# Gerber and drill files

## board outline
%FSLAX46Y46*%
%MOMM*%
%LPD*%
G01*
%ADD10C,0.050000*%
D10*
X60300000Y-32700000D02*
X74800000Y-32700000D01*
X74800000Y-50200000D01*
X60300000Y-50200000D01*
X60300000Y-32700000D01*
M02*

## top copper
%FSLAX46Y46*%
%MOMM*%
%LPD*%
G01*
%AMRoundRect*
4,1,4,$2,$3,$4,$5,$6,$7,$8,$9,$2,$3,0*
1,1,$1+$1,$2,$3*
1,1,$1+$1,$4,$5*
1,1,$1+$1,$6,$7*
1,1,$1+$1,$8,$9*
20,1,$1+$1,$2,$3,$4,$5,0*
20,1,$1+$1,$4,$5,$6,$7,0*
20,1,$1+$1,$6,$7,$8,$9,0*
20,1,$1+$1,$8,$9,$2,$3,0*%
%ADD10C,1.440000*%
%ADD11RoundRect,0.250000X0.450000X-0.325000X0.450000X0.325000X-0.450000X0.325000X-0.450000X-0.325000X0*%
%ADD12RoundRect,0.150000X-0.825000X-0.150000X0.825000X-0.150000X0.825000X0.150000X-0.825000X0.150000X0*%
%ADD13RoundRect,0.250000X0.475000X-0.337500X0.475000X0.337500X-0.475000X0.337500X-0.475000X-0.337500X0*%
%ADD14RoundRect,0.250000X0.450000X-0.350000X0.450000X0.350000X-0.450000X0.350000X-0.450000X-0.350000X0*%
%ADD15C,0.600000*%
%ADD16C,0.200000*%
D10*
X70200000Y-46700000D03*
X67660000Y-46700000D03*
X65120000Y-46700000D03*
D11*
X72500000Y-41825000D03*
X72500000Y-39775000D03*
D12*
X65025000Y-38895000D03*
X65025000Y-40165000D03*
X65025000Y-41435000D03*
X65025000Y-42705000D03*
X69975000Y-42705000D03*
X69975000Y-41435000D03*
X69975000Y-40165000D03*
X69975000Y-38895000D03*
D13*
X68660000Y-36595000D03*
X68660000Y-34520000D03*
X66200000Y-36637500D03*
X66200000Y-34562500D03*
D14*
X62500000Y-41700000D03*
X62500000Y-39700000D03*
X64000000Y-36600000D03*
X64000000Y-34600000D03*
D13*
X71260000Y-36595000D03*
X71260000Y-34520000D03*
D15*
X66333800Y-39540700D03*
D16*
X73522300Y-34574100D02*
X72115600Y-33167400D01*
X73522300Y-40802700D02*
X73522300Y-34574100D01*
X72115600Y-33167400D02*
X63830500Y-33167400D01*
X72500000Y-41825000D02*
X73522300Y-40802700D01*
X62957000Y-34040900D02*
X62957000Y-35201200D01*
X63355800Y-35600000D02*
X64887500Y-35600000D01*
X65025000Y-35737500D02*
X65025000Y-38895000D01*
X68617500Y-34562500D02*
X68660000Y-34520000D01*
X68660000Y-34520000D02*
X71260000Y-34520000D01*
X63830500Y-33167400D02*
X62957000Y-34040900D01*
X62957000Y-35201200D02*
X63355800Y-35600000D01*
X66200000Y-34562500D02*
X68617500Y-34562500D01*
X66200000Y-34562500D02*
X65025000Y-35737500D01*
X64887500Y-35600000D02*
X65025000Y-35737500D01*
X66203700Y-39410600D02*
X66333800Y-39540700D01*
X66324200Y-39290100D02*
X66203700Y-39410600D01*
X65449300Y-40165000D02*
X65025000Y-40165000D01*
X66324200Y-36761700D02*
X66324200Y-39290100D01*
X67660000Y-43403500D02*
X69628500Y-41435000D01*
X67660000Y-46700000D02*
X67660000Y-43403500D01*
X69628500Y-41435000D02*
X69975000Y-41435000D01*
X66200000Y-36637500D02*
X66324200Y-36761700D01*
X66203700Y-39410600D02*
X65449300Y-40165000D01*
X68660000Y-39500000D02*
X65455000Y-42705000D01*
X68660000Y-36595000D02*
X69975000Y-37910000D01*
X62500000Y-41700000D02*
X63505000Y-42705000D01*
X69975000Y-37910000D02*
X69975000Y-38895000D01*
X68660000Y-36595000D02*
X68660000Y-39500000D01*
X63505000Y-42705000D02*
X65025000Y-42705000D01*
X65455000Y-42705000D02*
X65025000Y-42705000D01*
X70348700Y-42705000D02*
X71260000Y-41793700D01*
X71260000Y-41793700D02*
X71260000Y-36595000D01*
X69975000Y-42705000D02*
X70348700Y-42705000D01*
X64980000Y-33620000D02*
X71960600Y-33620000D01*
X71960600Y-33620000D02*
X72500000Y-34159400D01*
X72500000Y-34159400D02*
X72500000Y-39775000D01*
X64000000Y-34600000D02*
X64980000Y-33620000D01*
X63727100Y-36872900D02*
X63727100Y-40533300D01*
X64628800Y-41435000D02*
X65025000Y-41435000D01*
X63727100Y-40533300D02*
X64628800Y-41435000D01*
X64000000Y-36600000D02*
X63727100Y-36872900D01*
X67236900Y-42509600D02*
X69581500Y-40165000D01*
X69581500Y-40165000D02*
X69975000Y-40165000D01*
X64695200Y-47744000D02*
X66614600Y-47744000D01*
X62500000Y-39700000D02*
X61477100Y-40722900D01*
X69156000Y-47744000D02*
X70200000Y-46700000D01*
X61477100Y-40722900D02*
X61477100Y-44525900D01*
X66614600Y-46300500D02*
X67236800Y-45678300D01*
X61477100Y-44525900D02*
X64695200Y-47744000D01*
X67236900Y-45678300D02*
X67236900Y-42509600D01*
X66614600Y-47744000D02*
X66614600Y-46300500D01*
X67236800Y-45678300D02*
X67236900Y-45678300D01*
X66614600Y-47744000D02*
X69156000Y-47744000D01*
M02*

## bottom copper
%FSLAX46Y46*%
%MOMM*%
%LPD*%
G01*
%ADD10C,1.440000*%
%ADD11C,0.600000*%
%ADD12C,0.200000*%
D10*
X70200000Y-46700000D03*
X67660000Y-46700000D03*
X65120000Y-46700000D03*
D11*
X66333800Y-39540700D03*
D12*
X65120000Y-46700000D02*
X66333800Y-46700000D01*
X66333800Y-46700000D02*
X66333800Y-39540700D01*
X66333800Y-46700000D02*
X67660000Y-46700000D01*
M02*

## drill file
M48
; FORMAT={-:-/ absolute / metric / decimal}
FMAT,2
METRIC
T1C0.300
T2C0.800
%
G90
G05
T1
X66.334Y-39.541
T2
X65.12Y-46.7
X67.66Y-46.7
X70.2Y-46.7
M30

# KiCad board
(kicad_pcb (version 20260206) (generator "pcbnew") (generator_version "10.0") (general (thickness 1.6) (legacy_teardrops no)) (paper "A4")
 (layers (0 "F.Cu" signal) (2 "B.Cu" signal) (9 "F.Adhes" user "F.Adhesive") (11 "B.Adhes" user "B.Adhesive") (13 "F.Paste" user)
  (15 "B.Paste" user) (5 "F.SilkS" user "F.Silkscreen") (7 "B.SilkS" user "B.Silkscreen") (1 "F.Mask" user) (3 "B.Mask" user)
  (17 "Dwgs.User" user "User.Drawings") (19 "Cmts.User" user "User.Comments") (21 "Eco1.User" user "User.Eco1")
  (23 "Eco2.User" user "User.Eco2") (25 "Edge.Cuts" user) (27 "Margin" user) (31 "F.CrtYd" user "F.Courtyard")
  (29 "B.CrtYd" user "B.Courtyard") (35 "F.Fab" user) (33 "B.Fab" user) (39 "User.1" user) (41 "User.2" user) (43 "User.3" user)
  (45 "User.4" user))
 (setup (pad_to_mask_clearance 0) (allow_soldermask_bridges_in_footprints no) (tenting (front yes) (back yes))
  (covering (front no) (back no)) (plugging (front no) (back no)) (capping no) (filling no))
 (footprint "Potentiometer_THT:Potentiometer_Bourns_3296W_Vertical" (layer "F.Cu") (at 70.2 46.7)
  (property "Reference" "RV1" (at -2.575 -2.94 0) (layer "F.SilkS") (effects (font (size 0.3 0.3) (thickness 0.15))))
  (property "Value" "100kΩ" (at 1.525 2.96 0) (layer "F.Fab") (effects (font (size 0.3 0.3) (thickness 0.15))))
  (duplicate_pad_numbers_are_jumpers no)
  (pad "1" thru_hole circle (at 0 0) (size 1.44 1.44) (drill 0.8) (layers "*.Cu" "*.Mask") (remove_unused_layers no) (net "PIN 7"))
  (pad "2" thru_hole circle (at -2.54 0) (size 1.44 1.44) (drill 0.8) (layers "*.Cu" "*.Mask") (remove_unused_layers no) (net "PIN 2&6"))
  (pad "3" thru_hole circle (at -5.08 0) (size 1.44 1.44) (drill 0.8) (layers "*.Cu" "*.Mask") (remove_unused_layers no) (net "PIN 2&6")))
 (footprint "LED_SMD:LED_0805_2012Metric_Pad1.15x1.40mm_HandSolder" (layer "F.Cu") (at 72.5 40.8 90)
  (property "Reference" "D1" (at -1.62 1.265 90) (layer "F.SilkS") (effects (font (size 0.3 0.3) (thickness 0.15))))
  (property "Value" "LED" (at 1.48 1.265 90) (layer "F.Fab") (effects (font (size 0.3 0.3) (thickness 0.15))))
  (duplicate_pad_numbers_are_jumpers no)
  (pad "1" smd roundrect (at -1.025 0 90) (size 1.15 1.4) (layers "F.Cu" "F.Mask" "F.Paste") (roundrect_rratio 0.217391) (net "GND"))
  (pad "2" smd roundrect (at 1.025 0 90) (size 1.15 1.4) (layers "F.Cu" "F.Mask" "F.Paste") (roundrect_rratio 0.217391) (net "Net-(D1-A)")))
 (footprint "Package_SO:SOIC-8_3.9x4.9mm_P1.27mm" (layer "F.Cu") (at 67.5 40.8)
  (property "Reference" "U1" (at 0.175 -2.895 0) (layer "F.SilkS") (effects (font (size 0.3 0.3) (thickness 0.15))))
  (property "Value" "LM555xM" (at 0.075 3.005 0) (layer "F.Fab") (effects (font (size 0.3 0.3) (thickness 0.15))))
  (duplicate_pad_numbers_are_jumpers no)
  (pad "1" smd roundrect (at -2.475 -1.905) (size 1.95 0.6) (layers "F.Cu" "F.Mask" "F.Paste") (roundrect_rratio 0.25) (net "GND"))
  (pad "2" smd roundrect (at -2.475 -0.635) (size 1.95 0.6) (layers "F.Cu" "F.Mask" "F.Paste") (roundrect_rratio 0.25) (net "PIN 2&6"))
  (pad "3" smd roundrect (at -2.475 0.635) (size 1.95 0.6) (layers "F.Cu" "F.Mask" "F.Paste") (roundrect_rratio 0.25) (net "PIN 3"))
  (pad "4" smd roundrect (at -2.475 1.905) (size 1.95 0.6) (layers "F.Cu" "F.Mask" "F.Paste") (roundrect_rratio 0.25) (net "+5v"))
  (pad "5" smd roundrect (at 2.475 1.905) (size 1.95 0.6) (layers "F.Cu" "F.Mask" "F.Paste") (roundrect_rratio 0.25) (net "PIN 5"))
  (pad "6" smd roundrect (at 2.475 0.635) (size 1.95 0.6) (layers "F.Cu" "F.Mask" "F.Paste") (roundrect_rratio 0.25) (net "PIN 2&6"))
  (pad "7" smd roundrect (at 2.475 -0.635) (size 1.95 0.6) (layers "F.Cu" "F.Mask" "F.Paste") (roundrect_rratio 0.25) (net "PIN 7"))
  (pad "8" smd roundrect (at 2.475 -1.905) (size 1.95 0.6) (layers "F.Cu" "F.Mask" "F.Paste") (roundrect_rratio 0.25) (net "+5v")))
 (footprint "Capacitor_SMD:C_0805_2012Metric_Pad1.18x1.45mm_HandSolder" (layer "F.Cu") (at 68.66 35.5575 90)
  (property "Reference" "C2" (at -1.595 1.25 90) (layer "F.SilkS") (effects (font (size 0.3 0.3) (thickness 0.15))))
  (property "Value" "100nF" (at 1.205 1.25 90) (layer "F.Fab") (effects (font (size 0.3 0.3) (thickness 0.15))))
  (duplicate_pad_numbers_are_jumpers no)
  (pad "1" smd roundrect (at -1.0375 0 90) (size 1.175 1.45) (layers "F.Cu" "F.Mask" "F.Paste") (roundrect_rratio 0.212766) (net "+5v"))
  (pad "2" smd roundrect (at 1.0375 0 90) (size 1.175 1.45) (layers "F.Cu" "F.Mask" "F.Paste") (roundrect_rratio 0.212766) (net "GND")))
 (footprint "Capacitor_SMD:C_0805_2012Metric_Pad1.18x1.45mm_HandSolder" (layer "F.Cu") (at 66.2 35.6 90)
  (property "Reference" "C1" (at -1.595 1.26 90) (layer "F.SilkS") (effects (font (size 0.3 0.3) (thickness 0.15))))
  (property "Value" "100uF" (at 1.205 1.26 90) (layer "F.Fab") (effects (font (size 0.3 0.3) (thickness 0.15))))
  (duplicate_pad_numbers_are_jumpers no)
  (pad "1" smd roundrect (at -1.0375 0 90) (size 1.175 1.45) (layers "F.Cu" "F.Mask" "F.Paste") (roundrect_rratio 0.212766) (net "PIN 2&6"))
  (pad "2" smd roundrect (at 1.0375 0 90) (size 1.175 1.45) (layers "F.Cu" "F.Mask" "F.Paste") (roundrect_rratio 0.212766) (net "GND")))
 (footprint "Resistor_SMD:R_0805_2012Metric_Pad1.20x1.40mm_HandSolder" (layer "F.Cu") (at 62.5 40.7 90)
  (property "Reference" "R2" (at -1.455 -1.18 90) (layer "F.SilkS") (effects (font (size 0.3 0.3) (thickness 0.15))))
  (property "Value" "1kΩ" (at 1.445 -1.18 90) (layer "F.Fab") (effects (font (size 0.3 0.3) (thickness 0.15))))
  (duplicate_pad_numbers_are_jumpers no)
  (pad "1" smd roundrect (at -1 0 90) (size 1.2 1.4) (layers "F.Cu" "F.Mask" "F.Paste") (roundrect_rratio 0.208333) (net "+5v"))
  (pad "2" smd roundrect (at 1 0 90) (size 1.2 1.4) (layers "F.Cu" "F.Mask" "F.Paste") (roundrect_rratio 0.208333) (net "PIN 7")))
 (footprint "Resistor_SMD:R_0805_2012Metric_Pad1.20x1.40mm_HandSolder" (layer "F.Cu") (at 64 35.6 90)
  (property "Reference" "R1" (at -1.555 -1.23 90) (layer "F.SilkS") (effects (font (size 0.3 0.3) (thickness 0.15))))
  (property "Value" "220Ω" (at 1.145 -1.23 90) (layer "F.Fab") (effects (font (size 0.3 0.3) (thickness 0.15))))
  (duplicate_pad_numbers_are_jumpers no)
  (pad "1" smd roundrect (at -1 0 90) (size 1.2 1.4) (layers "F.Cu" "F.Mask" "F.Paste") (roundrect_rratio 0.208333) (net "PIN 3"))
  (pad "2" smd roundrect (at 1 0 90) (size 1.2 1.4) (layers "F.Cu" "F.Mask" "F.Paste") (roundrect_rratio 0.208333) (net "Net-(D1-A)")))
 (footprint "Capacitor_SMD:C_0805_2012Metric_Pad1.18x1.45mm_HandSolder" (layer "F.Cu") (at 71.26 35.5575 90)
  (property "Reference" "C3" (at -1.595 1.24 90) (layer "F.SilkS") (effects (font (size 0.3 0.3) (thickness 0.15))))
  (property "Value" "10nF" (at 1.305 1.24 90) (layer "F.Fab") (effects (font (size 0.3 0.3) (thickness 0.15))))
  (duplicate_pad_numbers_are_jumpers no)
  (pad "1" smd roundrect (at -1.0375 0 90) (size 1.175 1.45) (layers "F.Cu" "F.Mask" "F.Paste") (roundrect_rratio 0.212766) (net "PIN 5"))
  (pad "2" smd roundrect (at 1.0375 0 90) (size 1.175 1.45) (layers "F.Cu" "F.Mask" "F.Paste") (roundrect_rratio 0.212766) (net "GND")))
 (gr_rect (start 60.3 32.7) (end 74.8 50.2) (stroke (width 0.05) (type default)) (fill no) (layer "Edge.Cuts"))
 (segment (start 73.5223 34.5741) (end 72.1156 33.1674) (width 0.2) (layer "F.Cu") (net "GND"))
 (segment (start 73.5223 40.8027) (end 73.5223 34.5741) (width 0.2) (layer "F.Cu") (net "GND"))
 (segment (start 72.1156 33.1674) (end 63.8305 33.1674) (width 0.2) (layer "F.Cu") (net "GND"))
 (segment (start 72.5 41.825) (end 73.5223 40.8027) (width 0.2) (layer "F.Cu") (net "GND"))
 (segment (start 62.957 34.0409) (end 62.957 35.2012) (width 0.2) (layer "F.Cu") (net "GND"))
 (segment (start 63.3558 35.6) (end 64.8875 35.6) (width 0.2) (layer "F.Cu") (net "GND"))
 (segment (start 65.025 35.7375) (end 65.025 38.895) (width 0.2) (layer "F.Cu") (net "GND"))
 (segment (start 68.6175 34.5625) (end 68.66 34.52) (width 0.2) (layer "F.Cu") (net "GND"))
 (segment (start 68.66 34.52) (end 71.26 34.52) (width 0.2) (layer "F.Cu") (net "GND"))
 (segment (start 63.8305 33.1674) (end 62.957 34.0409) (width 0.2) (layer "F.Cu") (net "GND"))
 (segment (start 62.957 35.2012) (end 63.3558 35.6) (width 0.2) (layer "F.Cu") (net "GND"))
 (segment (start 66.2 34.5625) (end 68.6175 34.5625) (width 0.2) (layer "F.Cu") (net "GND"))
 (segment (start 66.2 34.5625) (end 65.025 35.7375) (width 0.2) (layer "F.Cu") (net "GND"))
 (segment (start 64.8875 35.6) (end 65.025 35.7375) (width 0.2) (layer "F.Cu") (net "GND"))
 (segment (start 66.2037 39.4106) (end 66.3338 39.5407) (width 0.2) (layer "F.Cu") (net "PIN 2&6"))
 (segment (start 66.3242 39.2901) (end 66.2037 39.4106) (width 0.2) (layer "F.Cu") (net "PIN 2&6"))
 (segment (start 65.4493 40.165) (end 65.025 40.165) (width 0.2) (layer "F.Cu") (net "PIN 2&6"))
 (segment (start 66.3242 36.7617) (end 66.3242 39.2901) (width 0.2) (layer "F.Cu") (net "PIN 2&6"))
 (segment (start 67.66 43.4035) (end 69.6285 41.435) (width 0.2) (layer "F.Cu") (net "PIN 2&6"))
 (segment (start 67.66 46.7) (end 67.66 43.4035) (width 0.2) (layer "F.Cu") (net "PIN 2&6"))
 (segment (start 69.6285 41.435) (end 69.975 41.435) (width 0.2) (layer "F.Cu") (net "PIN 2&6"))
 (segment (start 66.2 36.6375) (end 66.3242 36.7617) (width 0.2) (layer "F.Cu") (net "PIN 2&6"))
 (segment (start 66.2037 39.4106) (end 65.4493 40.165) (width 0.2) (layer "F.Cu") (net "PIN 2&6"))
 (via (at 66.3338 39.5407) (size 0.6) (drill 0.3) (layers "F.Cu" "B.Cu") (capping no) (covering (front no) (back no))
  (plugging (front no) (back no)) (filling no) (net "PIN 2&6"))
 (segment (start 65.12 46.7) (end 66.3338 46.7) (width 0.2) (layer "B.Cu") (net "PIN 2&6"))
 (segment (start 66.3338 46.7) (end 66.3338 39.5407) (width 0.2) (layer "B.Cu") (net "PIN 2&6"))
 (segment (start 66.3338 46.7) (end 67.66 46.7) (width 0.2) (layer "B.Cu") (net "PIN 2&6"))
 (segment (start 68.66 39.5) (end 65.455 42.705) (width 0.2) (layer "F.Cu") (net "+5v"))
 (segment (start 68.66 36.595) (end 69.975 37.91) (width 0.2) (layer "F.Cu") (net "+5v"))
 (segment (start 62.5 41.7) (end 63.505 42.705) (width 0.2) (layer "F.Cu") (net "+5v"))
 (segment (start 69.975 37.91) (end 69.975 38.895) (width 0.2) (layer "F.Cu") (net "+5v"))
 (segment (start 68.66 36.595) (end 68.66 39.5) (width 0.2) (layer "F.Cu") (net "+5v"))
 (segment (start 63.505 42.705) (end 65.025 42.705) (width 0.2) (layer "F.Cu") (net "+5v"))
 (segment (start 65.455 42.705) (end 65.025 42.705) (width 0.2) (layer "F.Cu") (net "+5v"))
 (segment (start 70.3487 42.705) (end 71.26 41.7937) (width 0.2) (layer "F.Cu") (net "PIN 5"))
 (segment (start 71.26 41.7937) (end 71.26 36.595) (width 0.2) (layer "F.Cu") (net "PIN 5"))
 (segment (start 69.975 42.705) (end 70.3487 42.705) (width 0.2) (layer "F.Cu") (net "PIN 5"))
 (segment (start 64.98 33.62) (end 71.9606 33.62) (width 0.2) (layer "F.Cu") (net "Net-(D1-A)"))
 (segment (start 71.9606 33.62) (end 72.5 34.1594) (width 0.2) (layer "F.Cu") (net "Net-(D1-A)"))
 (segment (start 72.5 34.1594) (end 72.5 39.775) (width 0.2) (layer "F.Cu") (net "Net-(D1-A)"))
 (segment (start 64 34.6) (end 64.98 33.62) (width 0.2) (layer "F.Cu") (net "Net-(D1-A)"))
 (segment (start 63.7271 36.8729) (end 63.7271 40.5333) (width 0.2) (layer "F.Cu") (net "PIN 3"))
 (segment (start 64.6288 41.435) (end 65.025 41.435) (width 0.2) (layer "F.Cu") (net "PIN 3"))
 (segment (start 63.7271 40.5333) (end 64.6288 41.435) (width 0.2) (layer "F.Cu") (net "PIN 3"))
 (segment (start 64 36.6) (end 63.7271 36.8729) (width 0.2) (layer "F.Cu") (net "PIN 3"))
 (segment (start 67.2369 42.5096) (end 69.5815 40.165) (width 0.2) (layer "F.Cu") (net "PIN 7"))
 (segment (start 69.5815 40.165) (end 69.975 40.165) (width 0.2) (layer "F.Cu") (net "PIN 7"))
 (segment (start 64.6952 47.744) (end 66.6146 47.744) (width 0.2) (layer "F.Cu") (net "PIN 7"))
 (segment (start 62.5 39.7) (end 61.4771 40.7229) (width 0.2) (layer "F.Cu") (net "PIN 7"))
 (segment (start 69.156 47.744) (end 70.2 46.7) (width 0.2) (layer "F.Cu") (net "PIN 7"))
 (segment (start 61.4771 40.7229) (end 61.4771 44.5259) (width 0.2) (layer "F.Cu") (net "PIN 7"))
 (segment (start 66.6146 46.3005) (end 67.2368 45.6783) (width 0.2) (layer "F.Cu") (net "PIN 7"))
 (segment (start 61.4771 44.5259) (end 64.6952 47.744) (width 0.2) (layer "F.Cu") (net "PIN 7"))
 (segment (start 67.2369 45.6783) (end 67.2369 42.5096) (width 0.2) (layer "F.Cu") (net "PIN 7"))
 (segment (start 66.6146 47.744) (end 66.6146 46.3005) (width 0.2) (layer "F.Cu") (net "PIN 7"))
 (segment (start 67.2368 45.6783) (end 67.2369 45.6783) (width 0.2) (layer "F.Cu") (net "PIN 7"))
 (segment (start 66.6146 47.744) (end 69.156 47.744) (width 0.2) (layer "F.Cu") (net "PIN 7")))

